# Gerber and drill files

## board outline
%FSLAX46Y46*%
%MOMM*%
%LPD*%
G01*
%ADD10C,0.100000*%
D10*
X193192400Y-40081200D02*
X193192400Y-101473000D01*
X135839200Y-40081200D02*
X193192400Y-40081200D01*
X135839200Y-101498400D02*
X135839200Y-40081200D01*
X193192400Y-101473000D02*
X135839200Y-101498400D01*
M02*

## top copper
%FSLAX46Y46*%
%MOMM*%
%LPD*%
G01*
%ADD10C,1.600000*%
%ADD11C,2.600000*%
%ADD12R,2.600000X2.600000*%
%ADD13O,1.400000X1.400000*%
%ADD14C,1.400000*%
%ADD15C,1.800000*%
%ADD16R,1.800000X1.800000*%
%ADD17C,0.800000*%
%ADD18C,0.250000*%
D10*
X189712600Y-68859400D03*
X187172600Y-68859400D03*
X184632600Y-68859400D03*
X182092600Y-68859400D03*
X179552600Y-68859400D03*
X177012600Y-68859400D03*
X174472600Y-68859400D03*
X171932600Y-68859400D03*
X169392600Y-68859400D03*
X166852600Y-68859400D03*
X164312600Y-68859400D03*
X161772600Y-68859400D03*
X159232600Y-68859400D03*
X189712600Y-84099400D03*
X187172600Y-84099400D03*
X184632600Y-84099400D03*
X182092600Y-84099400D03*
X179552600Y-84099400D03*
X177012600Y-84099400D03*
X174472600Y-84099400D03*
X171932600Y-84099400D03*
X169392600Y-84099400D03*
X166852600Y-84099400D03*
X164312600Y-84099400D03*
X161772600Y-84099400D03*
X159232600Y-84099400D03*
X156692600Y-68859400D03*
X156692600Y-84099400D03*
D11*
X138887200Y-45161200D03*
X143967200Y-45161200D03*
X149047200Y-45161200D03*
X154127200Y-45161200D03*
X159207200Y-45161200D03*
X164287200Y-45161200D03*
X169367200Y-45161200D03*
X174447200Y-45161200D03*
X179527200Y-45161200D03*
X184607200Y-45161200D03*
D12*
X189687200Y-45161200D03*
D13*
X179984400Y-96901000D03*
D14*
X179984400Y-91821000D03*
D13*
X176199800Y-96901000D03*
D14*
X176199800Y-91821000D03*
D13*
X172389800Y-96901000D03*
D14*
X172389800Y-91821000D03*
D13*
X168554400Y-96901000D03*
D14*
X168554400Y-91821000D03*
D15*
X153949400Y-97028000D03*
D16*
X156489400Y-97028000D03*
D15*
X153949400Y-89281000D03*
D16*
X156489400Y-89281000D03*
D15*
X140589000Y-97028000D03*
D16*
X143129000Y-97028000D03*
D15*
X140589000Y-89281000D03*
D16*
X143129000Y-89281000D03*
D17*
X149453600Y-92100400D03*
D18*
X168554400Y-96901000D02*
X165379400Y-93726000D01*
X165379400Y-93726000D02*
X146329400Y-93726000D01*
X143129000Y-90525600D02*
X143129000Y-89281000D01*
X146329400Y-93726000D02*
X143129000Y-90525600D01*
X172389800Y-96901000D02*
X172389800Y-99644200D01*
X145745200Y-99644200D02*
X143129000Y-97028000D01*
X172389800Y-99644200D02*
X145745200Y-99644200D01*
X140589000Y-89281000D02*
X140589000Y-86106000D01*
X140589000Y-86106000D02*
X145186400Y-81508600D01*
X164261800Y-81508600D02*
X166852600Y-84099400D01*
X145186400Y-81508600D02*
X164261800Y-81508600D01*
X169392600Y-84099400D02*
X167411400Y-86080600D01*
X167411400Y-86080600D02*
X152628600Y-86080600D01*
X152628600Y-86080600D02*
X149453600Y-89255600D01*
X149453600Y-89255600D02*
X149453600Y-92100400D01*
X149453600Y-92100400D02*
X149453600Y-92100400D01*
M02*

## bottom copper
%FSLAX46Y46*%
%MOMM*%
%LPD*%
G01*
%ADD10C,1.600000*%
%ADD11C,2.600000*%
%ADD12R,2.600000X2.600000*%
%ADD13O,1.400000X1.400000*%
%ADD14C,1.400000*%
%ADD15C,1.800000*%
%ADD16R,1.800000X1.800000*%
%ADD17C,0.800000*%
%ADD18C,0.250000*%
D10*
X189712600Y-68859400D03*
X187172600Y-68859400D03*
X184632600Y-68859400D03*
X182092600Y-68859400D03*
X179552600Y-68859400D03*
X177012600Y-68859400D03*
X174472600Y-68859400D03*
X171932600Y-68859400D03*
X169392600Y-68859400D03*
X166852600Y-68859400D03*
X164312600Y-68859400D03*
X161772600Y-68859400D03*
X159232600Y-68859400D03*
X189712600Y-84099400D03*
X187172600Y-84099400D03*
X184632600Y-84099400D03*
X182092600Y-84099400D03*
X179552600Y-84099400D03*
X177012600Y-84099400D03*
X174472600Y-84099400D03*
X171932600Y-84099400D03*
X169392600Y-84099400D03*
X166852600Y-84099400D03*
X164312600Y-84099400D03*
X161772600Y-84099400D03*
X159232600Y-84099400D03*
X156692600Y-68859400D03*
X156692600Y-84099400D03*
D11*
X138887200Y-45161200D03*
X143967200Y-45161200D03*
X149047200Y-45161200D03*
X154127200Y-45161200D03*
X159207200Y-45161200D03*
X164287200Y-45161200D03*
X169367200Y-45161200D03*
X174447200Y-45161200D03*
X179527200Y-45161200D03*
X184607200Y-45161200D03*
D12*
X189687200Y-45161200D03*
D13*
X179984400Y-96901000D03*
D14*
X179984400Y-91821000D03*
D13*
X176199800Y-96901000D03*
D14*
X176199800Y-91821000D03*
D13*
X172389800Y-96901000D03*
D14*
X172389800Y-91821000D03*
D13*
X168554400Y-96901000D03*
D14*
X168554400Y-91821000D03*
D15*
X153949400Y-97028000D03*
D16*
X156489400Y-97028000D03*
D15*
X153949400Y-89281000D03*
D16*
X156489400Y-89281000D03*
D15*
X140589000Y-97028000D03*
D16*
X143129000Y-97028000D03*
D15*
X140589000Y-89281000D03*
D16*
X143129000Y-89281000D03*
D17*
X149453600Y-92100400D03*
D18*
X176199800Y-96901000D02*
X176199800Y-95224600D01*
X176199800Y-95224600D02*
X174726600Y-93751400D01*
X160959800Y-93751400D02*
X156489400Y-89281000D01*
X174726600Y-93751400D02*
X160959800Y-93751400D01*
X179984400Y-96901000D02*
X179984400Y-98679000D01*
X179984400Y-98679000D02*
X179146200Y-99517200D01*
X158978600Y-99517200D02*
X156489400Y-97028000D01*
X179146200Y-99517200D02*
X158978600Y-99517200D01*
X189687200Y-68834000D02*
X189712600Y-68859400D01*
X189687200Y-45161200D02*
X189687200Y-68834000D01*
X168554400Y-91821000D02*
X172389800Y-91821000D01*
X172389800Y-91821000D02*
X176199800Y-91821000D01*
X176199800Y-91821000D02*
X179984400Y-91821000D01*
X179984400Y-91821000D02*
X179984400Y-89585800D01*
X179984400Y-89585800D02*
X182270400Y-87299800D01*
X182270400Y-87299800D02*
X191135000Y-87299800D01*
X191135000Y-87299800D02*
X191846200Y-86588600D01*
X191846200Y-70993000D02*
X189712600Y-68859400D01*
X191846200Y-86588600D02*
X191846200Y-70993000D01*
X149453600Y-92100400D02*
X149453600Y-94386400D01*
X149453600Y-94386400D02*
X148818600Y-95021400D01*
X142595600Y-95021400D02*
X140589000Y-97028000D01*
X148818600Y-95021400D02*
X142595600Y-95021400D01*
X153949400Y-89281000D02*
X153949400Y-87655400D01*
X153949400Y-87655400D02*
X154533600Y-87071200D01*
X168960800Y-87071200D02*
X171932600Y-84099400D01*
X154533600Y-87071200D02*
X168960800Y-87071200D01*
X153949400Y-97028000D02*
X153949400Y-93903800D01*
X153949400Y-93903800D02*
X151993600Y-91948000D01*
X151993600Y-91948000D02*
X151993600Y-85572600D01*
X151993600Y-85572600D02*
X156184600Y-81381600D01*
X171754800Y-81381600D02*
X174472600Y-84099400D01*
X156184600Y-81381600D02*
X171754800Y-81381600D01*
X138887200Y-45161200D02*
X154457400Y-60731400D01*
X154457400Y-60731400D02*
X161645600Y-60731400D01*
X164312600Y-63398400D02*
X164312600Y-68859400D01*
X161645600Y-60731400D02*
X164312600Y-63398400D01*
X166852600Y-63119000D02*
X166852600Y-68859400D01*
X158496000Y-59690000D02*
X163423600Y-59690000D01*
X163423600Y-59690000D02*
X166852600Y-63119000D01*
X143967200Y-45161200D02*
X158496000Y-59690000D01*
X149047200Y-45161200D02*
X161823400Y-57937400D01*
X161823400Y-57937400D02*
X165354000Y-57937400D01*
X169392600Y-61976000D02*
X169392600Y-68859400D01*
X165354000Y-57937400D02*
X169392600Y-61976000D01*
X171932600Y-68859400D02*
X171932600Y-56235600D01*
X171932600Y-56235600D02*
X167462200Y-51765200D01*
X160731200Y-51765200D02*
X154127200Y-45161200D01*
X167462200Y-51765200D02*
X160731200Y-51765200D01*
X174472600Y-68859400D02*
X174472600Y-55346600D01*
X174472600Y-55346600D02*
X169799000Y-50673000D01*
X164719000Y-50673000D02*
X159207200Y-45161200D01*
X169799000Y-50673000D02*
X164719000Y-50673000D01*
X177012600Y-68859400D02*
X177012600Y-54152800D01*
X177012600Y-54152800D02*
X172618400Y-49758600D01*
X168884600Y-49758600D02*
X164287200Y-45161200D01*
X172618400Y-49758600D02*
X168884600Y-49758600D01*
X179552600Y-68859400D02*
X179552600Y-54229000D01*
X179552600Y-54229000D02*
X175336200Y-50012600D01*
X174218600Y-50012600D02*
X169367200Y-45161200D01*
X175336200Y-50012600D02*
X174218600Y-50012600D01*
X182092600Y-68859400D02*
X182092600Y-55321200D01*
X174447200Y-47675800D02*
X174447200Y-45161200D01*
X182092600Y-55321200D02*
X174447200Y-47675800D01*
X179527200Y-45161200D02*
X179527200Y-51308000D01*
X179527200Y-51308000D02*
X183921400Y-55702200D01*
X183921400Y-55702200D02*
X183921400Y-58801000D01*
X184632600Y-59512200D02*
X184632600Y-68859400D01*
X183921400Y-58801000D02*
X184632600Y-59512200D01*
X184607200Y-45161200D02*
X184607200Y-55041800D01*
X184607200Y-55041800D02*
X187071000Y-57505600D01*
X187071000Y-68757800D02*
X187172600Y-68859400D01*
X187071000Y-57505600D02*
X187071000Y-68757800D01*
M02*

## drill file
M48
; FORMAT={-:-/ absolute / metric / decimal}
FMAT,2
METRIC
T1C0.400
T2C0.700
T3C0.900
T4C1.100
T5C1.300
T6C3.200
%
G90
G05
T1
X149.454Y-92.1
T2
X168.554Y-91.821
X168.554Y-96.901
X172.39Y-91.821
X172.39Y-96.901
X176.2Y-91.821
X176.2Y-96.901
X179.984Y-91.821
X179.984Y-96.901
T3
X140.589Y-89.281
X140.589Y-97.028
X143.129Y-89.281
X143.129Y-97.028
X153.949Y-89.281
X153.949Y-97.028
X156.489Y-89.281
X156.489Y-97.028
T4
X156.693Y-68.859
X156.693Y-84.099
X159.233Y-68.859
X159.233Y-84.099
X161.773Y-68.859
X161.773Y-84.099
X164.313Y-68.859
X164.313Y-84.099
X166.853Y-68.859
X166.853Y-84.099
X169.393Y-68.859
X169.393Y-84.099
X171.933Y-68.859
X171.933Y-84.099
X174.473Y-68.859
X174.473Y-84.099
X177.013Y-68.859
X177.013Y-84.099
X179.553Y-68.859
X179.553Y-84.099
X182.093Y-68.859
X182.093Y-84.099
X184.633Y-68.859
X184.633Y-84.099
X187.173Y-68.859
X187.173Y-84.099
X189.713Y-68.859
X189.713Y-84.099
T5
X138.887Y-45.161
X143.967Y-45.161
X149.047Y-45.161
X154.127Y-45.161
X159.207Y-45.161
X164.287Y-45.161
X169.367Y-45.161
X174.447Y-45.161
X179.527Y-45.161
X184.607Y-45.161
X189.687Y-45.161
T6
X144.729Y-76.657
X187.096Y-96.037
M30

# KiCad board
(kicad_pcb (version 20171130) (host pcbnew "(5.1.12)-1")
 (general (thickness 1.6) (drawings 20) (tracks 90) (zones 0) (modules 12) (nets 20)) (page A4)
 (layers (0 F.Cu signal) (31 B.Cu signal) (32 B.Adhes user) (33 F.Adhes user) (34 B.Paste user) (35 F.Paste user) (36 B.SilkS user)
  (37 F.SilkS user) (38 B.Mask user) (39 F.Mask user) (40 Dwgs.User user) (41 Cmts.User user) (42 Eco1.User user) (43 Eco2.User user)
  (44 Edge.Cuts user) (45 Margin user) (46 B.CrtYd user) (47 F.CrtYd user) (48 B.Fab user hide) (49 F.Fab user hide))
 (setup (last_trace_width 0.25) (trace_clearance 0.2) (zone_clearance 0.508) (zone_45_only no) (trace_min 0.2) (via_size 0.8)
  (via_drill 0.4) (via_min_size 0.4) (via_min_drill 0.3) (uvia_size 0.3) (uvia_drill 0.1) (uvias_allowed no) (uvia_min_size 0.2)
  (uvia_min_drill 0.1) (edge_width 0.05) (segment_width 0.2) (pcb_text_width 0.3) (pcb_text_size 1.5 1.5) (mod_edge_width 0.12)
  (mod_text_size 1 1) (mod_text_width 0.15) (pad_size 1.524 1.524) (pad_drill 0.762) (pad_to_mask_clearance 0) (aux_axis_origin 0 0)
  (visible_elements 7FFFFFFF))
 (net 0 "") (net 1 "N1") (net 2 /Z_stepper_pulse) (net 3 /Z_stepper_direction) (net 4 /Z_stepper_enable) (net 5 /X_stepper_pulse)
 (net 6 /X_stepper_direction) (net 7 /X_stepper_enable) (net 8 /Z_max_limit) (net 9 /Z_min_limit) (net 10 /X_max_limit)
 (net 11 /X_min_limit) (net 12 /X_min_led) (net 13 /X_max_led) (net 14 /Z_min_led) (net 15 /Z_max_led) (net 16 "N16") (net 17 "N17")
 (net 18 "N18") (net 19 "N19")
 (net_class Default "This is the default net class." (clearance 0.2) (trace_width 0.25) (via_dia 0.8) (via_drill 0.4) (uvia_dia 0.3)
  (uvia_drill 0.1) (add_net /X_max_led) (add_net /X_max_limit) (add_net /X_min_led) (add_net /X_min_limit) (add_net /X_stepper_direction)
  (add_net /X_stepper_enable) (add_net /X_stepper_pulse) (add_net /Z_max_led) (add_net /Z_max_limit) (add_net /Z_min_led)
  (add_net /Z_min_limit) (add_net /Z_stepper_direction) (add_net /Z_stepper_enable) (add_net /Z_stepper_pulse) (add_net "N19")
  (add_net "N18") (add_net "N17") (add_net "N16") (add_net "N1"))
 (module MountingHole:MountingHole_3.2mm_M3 (layer F.Cu) (at 144.7292 76.6572)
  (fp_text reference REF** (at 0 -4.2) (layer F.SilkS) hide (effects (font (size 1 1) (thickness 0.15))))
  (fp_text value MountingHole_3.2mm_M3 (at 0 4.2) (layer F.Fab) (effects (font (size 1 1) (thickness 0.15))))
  (pad 1 np_thru_hole circle (at 0 0) (size 3.2 3.2) (drill 3.2) (layers *.Cu *.Mask)))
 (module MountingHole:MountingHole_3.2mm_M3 (layer F.Cu) (at 187.0964 96.0374)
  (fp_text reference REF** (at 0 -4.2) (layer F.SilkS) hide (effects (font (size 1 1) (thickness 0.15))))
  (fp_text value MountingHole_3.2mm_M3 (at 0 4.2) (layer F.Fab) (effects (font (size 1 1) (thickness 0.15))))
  (pad 1 np_thru_hole circle (at 0 0) (size 3.2 3.2) (drill 3.2) (layers *.Cu *.Mask)))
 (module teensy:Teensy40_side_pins (layer F.Cu) (at 173.2026 76.4794 180)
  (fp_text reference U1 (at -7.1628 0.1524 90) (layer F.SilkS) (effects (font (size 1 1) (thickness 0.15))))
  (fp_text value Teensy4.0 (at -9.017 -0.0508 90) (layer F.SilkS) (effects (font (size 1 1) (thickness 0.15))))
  (pad 1 thru_hole circle (at -16.51 7.62 180) (size 1.6 1.6) (drill 1.1) (layers *.Cu *.Mask) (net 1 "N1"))
  (pad 2 thru_hole circle (at -13.97 7.62 180) (size 1.6 1.6) (drill 1.1) (layers *.Cu *.Mask) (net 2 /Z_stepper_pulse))
  (pad 3 thru_hole circle (at -11.43 7.62 180) (size 1.6 1.6) (drill 1.1) (layers *.Cu *.Mask) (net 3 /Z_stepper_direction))
  (pad 4 thru_hole circle (at -8.89 7.62 180) (size 1.6 1.6) (drill 1.1) (layers *.Cu *.Mask) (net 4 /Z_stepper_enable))
  (pad 5 thru_hole circle (at -6.35 7.62 180) (size 1.6 1.6) (drill 1.1) (layers *.Cu *.Mask) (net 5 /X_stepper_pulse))
  (pad 6 thru_hole circle (at -3.81 7.62 180) (size 1.6 1.6) (drill 1.1) (layers *.Cu *.Mask) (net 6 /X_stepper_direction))
  (pad 7 thru_hole circle (at -1.27 7.62 180) (size 1.6 1.6) (drill 1.1) (layers *.Cu *.Mask) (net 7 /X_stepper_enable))
  (pad 8 thru_hole circle (at 1.27 7.62 180) (size 1.6 1.6) (drill 1.1) (layers *.Cu *.Mask) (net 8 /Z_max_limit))
  (pad 9 thru_hole circle (at 3.81 7.62 180) (size 1.6 1.6) (drill 1.1) (layers *.Cu *.Mask) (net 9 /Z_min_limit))
  (pad 10 thru_hole circle (at 6.35 7.62 180) (size 1.6 1.6) (drill 1.1) (layers *.Cu *.Mask) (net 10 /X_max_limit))
  (pad 11 thru_hole circle (at 8.89 7.62 180) (size 1.6 1.6) (drill 1.1) (layers *.Cu *.Mask) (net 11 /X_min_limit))
  (pad 12 thru_hole circle (at 11.43 7.62 180) (size 1.6 1.6) (drill 1.1) (layers *.Cu *.Mask))
  (pad 13 thru_hole circle (at 13.97 7.62 180) (size 1.6 1.6) (drill 1.1) (layers *.Cu *.Mask))
  (pad 33 thru_hole circle (at -16.51 -7.62 180) (size 1.6 1.6) (drill 1.1) (layers *.Cu *.Mask))
  (pad 32 thru_hole circle (at -13.97 -7.62 180) (size 1.6 1.6) (drill 1.1) (layers *.Cu *.Mask))
  (pad 31 thru_hole circle (at -11.43 -7.62 180) (size 1.6 1.6) (drill 1.1) (layers *.Cu *.Mask))
  (pad 30 thru_hole circle (at -8.89 -7.62 180) (size 1.6 1.6) (drill 1.1) (layers *.Cu *.Mask))
  (pad 29 thru_hole circle (at -6.35 -7.62 180) (size 1.6 1.6) (drill 1.1) (layers *.Cu *.Mask))
  (pad 28 thru_hole circle (at -3.81 -7.62 180) (size 1.6 1.6) (drill 1.1) (layers *.Cu *.Mask))
  (pad 27 thru_hole circle (at -1.27 -7.62 180) (size 1.6 1.6) (drill 1.1) (layers *.Cu *.Mask) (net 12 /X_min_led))
  (pad 26 thru_hole circle (at 1.27 -7.62 180) (size 1.6 1.6) (drill 1.1) (layers *.Cu *.Mask) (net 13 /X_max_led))
  (pad 25 thru_hole circle (at 3.81 -7.62 180) (size 1.6 1.6) (drill 1.1) (layers *.Cu *.Mask) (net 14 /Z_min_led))
  (pad 24 thru_hole circle (at 6.35 -7.62 180) (size 1.6 1.6) (drill 1.1) (layers *.Cu *.Mask) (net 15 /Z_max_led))
  (pad 23 thru_hole circle (at 8.89 -7.62 180) (size 1.6 1.6) (drill 1.1) (layers *.Cu *.Mask))
  (pad 22 thru_hole circle (at 11.43 -7.62 180) (size 1.6 1.6) (drill 1.1) (layers *.Cu *.Mask))
  (pad 21 thru_hole circle (at 13.97 -7.62 180) (size 1.6 1.6) (drill 1.1) (layers *.Cu *.Mask))
  (pad 14 thru_hole circle (at 16.51 7.62 180) (size 1.6 1.6) (drill 1.1) (layers *.Cu *.Mask))
  (pad 20 thru_hole circle (at 16.51 -7.62 180) (size 1.6 1.6) (drill 1.1) (layers *.Cu *.Mask)))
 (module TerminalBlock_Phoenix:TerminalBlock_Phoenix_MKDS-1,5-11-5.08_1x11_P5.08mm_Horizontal (layer F.Cu) (at 189.6872 45.1612 180)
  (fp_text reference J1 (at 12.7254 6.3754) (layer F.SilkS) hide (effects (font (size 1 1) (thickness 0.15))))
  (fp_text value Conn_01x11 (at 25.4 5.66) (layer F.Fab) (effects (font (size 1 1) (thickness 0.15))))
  (pad 11 thru_hole circle (at 50.8 0 180) (size 2.6 2.6) (drill 1.3) (layers *.Cu *.Mask) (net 11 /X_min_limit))
  (pad 10 thru_hole circle (at 45.72 0 180) (size 2.6 2.6) (drill 1.3) (layers *.Cu *.Mask) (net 10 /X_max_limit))
  (pad 9 thru_hole circle (at 40.64 0 180) (size 2.6 2.6) (drill 1.3) (layers *.Cu *.Mask) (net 9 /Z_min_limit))
  (pad 8 thru_hole circle (at 35.56 0 180) (size 2.6 2.6) (drill 1.3) (layers *.Cu *.Mask) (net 8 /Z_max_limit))
  (pad 7 thru_hole circle (at 30.48 0 180) (size 2.6 2.6) (drill 1.3) (layers *.Cu *.Mask) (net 7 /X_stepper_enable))
  (pad 6 thru_hole circle (at 25.4 0 180) (size 2.6 2.6) (drill 1.3) (layers *.Cu *.Mask) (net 6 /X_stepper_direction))
  (pad 5 thru_hole circle (at 20.32 0 180) (size 2.6 2.6) (drill 1.3) (layers *.Cu *.Mask) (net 5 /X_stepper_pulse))
  (pad 4 thru_hole circle (at 15.24 0 180) (size 2.6 2.6) (drill 1.3) (layers *.Cu *.Mask) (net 4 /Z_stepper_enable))
  (pad 3 thru_hole circle (at 10.16 0 180) (size 2.6 2.6) (drill 1.3) (layers *.Cu *.Mask) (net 3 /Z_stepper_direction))
  (pad 2 thru_hole circle (at 5.08 0 180) (size 2.6 2.6) (drill 1.3) (layers *.Cu *.Mask) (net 2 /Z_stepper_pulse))
  (pad 1 thru_hole rect (at 0 0 180) (size 2.6 2.6) (drill 1.3) (layers *.Cu *.Mask) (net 1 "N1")))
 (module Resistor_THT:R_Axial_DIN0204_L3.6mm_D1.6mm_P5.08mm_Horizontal (layer F.Cu) (at 179.9844 91.821 270)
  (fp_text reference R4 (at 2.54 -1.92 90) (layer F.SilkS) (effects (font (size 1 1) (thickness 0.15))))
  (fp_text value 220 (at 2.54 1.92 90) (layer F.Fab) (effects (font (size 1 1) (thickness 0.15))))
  (pad 2 thru_hole oval (at 5.08 0 270) (size 1.4 1.4) (drill 0.7) (layers *.Cu *.Mask) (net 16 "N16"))
  (pad 1 thru_hole circle (at 0 0 270) (size 1.4 1.4) (drill 0.7) (layers *.Cu *.Mask) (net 1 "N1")))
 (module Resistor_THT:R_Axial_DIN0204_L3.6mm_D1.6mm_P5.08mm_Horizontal (layer F.Cu) (at 176.1998 91.821 270)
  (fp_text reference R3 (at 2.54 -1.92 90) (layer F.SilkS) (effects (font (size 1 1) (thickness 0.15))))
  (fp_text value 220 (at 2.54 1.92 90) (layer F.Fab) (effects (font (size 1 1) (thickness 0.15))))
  (pad 2 thru_hole oval (at 5.08 0 270) (size 1.4 1.4) (drill 0.7) (layers *.Cu *.Mask) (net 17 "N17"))
  (pad 1 thru_hole circle (at 0 0 270) (size 1.4 1.4) (drill 0.7) (layers *.Cu *.Mask) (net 1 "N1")))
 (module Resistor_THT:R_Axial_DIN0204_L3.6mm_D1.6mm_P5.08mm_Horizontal (layer F.Cu) (at 172.3898 91.821 270)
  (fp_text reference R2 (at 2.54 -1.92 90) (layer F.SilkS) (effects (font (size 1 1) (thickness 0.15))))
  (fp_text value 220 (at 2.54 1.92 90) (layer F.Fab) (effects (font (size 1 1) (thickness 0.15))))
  (pad 2 thru_hole oval (at 5.08 0 270) (size 1.4 1.4) (drill 0.7) (layers *.Cu *.Mask) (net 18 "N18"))
  (pad 1 thru_hole circle (at 0 0 270) (size 1.4 1.4) (drill 0.7) (layers *.Cu *.Mask) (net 1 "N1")))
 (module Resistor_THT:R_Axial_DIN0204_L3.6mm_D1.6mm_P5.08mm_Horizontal (layer F.Cu) (at 168.5544 91.821 270)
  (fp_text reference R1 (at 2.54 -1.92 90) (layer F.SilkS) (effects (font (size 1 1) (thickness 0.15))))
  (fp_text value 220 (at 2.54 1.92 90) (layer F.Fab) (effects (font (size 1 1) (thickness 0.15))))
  (pad 2 thru_hole oval (at 5.08 0 270) (size 1.4 1.4) (drill 0.7) (layers *.Cu *.Mask) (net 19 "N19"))
  (pad 1 thru_hole circle (at 0 0 270) (size 1.4 1.4) (drill 0.7) (layers *.Cu *.Mask) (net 1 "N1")))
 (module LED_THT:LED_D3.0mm (layer F.Cu) (at 156.4894 97.028 180)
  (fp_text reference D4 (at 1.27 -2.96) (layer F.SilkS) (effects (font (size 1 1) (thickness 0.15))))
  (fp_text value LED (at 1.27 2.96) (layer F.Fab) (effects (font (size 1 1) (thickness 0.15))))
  (pad 2 thru_hole circle (at 2.54 0 180) (size 1.8 1.8) (drill 0.9) (layers *.Cu *.Mask) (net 12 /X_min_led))
  (pad 1 thru_hole rect (at 0 0 180) (size 1.8 1.8) (drill 0.9) (layers *.Cu *.Mask) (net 16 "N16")))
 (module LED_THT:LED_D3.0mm (layer F.Cu) (at 156.4894 89.281 180)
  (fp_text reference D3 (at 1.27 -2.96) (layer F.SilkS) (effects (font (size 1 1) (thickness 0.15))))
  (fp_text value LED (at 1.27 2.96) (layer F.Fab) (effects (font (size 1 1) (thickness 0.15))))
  (pad 2 thru_hole circle (at 2.54 0 180) (size 1.8 1.8) (drill 0.9) (layers *.Cu *.Mask) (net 13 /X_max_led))
  (pad 1 thru_hole rect (at 0 0 180) (size 1.8 1.8) (drill 0.9) (layers *.Cu *.Mask) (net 17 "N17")))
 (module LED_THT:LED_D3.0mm (layer F.Cu) (at 143.129 97.028 180)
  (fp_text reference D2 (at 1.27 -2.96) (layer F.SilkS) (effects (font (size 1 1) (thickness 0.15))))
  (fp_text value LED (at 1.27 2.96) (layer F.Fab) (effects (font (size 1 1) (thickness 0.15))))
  (pad 2 thru_hole circle (at 2.54 0 180) (size 1.8 1.8) (drill 0.9) (layers *.Cu *.Mask) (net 14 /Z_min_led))
  (pad 1 thru_hole rect (at 0 0 180) (size 1.8 1.8) (drill 0.9) (layers *.Cu *.Mask) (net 18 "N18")))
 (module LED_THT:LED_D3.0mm (layer F.Cu) (at 143.129 89.281 180)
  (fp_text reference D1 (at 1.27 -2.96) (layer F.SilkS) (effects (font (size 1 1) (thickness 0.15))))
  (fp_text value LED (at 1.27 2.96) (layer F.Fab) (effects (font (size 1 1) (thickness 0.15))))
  (pad 2 thru_hole circle (at 2.54 0 180) (size 1.8 1.8) (drill 0.9) (layers *.Cu *.Mask) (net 15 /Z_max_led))
  (pad 1 thru_hole rect (at 0 0 180) (size 1.8 1.8) (drill 0.9) (layers *.Cu *.Mask) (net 19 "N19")))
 (gr_line (start 193.1924 40.0812) (end 193.1924 101.473) (layer Edge.Cuts) (width 0.1))
 (gr_line (start 135.8392 40.0812) (end 193.1924 40.0812) (layer Edge.Cuts) (width 0.1))
 (gr_line (start 135.8392 101.4984) (end 135.8392 40.0812) (layer Edge.Cuts) (width 0.1))
 (gr_line (start 193.1924 101.473) (end 135.8392 101.4984) (layer Edge.Cuts) (width 0.1))
 (segment (start 168.5544 96.901) (end 165.3794 93.726) (width 0.25) (layer F.Cu) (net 19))
 (segment (start 165.3794 93.726) (end 146.3294 93.726) (width 0.25) (layer F.Cu) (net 19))
 (segment (start 143.129 90.5256) (end 143.129 89.281) (width 0.25) (layer F.Cu) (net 19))
 (segment (start 146.3294 93.726) (end 143.129 90.5256) (width 0.25) (layer F.Cu) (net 19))
 (segment (start 172.3898 96.901) (end 172.3898 99.6442) (width 0.25) (layer F.Cu) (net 18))
 (segment (start 145.7452 99.6442) (end 143.129 97.028) (width 0.25) (layer F.Cu) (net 18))
 (segment (start 172.3898 99.6442) (end 145.7452 99.6442) (width 0.25) (layer F.Cu) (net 18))
 (segment (start 176.1998 96.901) (end 176.1998 95.2246) (width 0.25) (layer B.Cu) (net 17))
 (segment (start 176.1998 95.2246) (end 174.7266 93.7514) (width 0.25) (layer B.Cu) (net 17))
 (segment (start 160.9598 93.7514) (end 156.4894 89.281) (width 0.25) (layer B.Cu) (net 17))
 (segment (start 174.7266 93.7514) (end 160.9598 93.7514) (width 0.25) (layer B.Cu) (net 17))
 (segment (start 179.9844 96.901) (end 179.9844 98.679) (width 0.25) (layer B.Cu) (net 16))
 (segment (start 179.9844 98.679) (end 179.1462 99.5172) (width 0.25) (layer B.Cu) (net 16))
 (segment (start 158.9786 99.5172) (end 156.4894 97.028) (width 0.25) (layer B.Cu) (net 16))
 (segment (start 179.1462 99.5172) (end 158.9786 99.5172) (width 0.25) (layer B.Cu) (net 16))
 (segment (start 189.6872 68.834) (end 189.7126 68.8594) (width 0.25) (layer B.Cu) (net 1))
 (segment (start 189.6872 45.1612) (end 189.6872 68.834) (width 0.25) (layer B.Cu) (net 1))
 (segment (start 168.5544 91.821) (end 172.3898 91.821) (width 0.25) (layer B.Cu) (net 1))
 (segment (start 172.3898 91.821) (end 176.1998 91.821) (width 0.25) (layer B.Cu) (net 1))
 (segment (start 176.1998 91.821) (end 179.9844 91.821) (width 0.25) (layer B.Cu) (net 1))
 (segment (start 179.9844 91.821) (end 179.9844 89.5858) (width 0.25) (layer B.Cu) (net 1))
 (segment (start 179.9844 89.5858) (end 182.2704 87.2998) (width 0.25) (layer B.Cu) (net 1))
 (segment (start 182.2704 87.2998) (end 191.135 87.2998) (width 0.25) (layer B.Cu) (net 1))
 (segment (start 191.135 87.2998) (end 191.8462 86.5886) (width 0.25) (layer B.Cu) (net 1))
 (segment (start 191.8462 70.993) (end 189.7126 68.8594) (width 0.25) (layer B.Cu) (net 1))
 (segment (start 191.8462 86.5886) (end 191.8462 70.993) (width 0.25) (layer B.Cu) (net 1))
 (segment (start 140.589 89.281) (end 140.589 86.106) (width 0.25) (layer F.Cu) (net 15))
 (segment (start 140.589 86.106) (end 145.1864 81.5086) (width 0.25) (layer F.Cu) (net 15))
 (segment (start 164.2618 81.5086) (end 166.8526 84.0994) (width 0.25) (layer F.Cu) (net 15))
 (segment (start 145.1864 81.5086) (end 164.2618 81.5086) (width 0.25) (layer F.Cu) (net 15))
 (segment (start 169.3926 84.0994) (end 167.4114 86.0806) (width 0.25) (layer F.Cu) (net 14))
 (segment (start 167.4114 86.0806) (end 152.6286 86.0806) (width 0.25) (layer F.Cu) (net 14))
 (segment (start 152.6286 86.0806) (end 149.4536 89.2556) (width 0.25) (layer F.Cu) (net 14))
 (segment (start 149.4536 89.2556) (end 149.4536 92.1004) (width 0.25) (layer F.Cu) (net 14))
 (segment (start 149.4536 92.1004) (end 149.4536 92.1004) (width 0.25) (layer F.Cu) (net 14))
 (via (at 149.4536 92.1004) (size 0.8) (drill 0.4) (layers F.Cu B.Cu) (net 14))
 (segment (start 149.4536 92.1004) (end 149.4536 94.3864) (width 0.25) (layer B.Cu) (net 14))
 (segment (start 149.4536 94.3864) (end 148.8186 95.0214) (width 0.25) (layer B.Cu) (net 14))
 (segment (start 142.5956 95.0214) (end 140.589 97.028) (width 0.25) (layer B.Cu) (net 14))
 (segment (start 148.8186 95.0214) (end 142.5956 95.0214) (width 0.25) (layer B.Cu) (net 14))
 (segment (start 153.9494 89.281) (end 153.9494 87.6554) (width 0.25) (layer B.Cu) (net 13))
 (segment (start 153.9494 87.6554) (end 154.5336 87.0712) (width 0.25) (layer B.Cu) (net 13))
 (segment (start 168.9608 87.0712) (end 171.9326 84.0994) (width 0.25) (layer B.Cu) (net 13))
 (segment (start 154.5336 87.0712) (end 168.9608 87.0712) (width 0.25) (layer B.Cu) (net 13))
 (segment (start 153.9494 97.028) (end 153.9494 93.9038) (width 0.25) (layer B.Cu) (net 12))
 (segment (start 153.9494 93.9038) (end 151.9936 91.948) (width 0.25) (layer B.Cu) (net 12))
 (segment (start 151.9936 91.948) (end 151.9936 85.5726) (width 0.25) (layer B.Cu) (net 12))
 (segment (start 151.9936 85.5726) (end 156.1846 81.3816) (width 0.25) (layer B.Cu) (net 12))
 (segment (start 171.7548 81.3816) (end 174.4726 84.0994) (width 0.25) (layer B.Cu) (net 12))
 (segment (start 156.1846 81.3816) (end 171.7548 81.3816) (width 0.25) (layer B.Cu) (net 12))
 (segment (start 138.8872 45.1612) (end 154.4574 60.7314) (width 0.25) (layer B.Cu) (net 11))
 (segment (start 154.4574 60.7314) (end 161.6456 60.7314) (width 0.25) (layer B.Cu) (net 11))
 (segment (start 164.3126 63.3984) (end 164.3126 68.8594) (width 0.25) (layer B.Cu) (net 11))
 (segment (start 161.6456 60.7314) (end 164.3126 63.3984) (width 0.25) (layer B.Cu) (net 11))
 (segment (start 166.8526 63.119) (end 166.8526 68.8594) (width 0.25) (layer B.Cu) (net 10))
 (segment (start 158.496 59.69) (end 163.4236 59.69) (width 0.25) (layer B.Cu) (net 10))
 (segment (start 163.4236 59.69) (end 166.8526 63.119) (width 0.25) (layer B.Cu) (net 10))
 (segment (start 143.9672 45.1612) (end 158.496 59.69) (width 0.25) (layer B.Cu) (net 10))
 (segment (start 149.0472 45.1612) (end 161.8234 57.9374) (width 0.25) (layer B.Cu) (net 9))
 (segment (start 161.8234 57.9374) (end 165.354 57.9374) (width 0.25) (layer B.Cu) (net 9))
 (segment (start 169.3926 61.976) (end 169.3926 68.8594) (width 0.25) (layer B.Cu) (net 9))
 (segment (start 165.354 57.9374) (end 169.3926 61.976) (width 0.25) (layer B.Cu) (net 9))
 (segment (start 171.9326 68.8594) (end 171.9326 56.2356) (width 0.25) (layer B.Cu) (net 8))
 (segment (start 171.9326 56.2356) (end 167.4622 51.7652) (width 0.25) (layer B.Cu) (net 8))
 (segment (start 160.7312 51.7652) (end 154.1272 45.1612) (width 0.25) (layer B.Cu) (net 8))
 (segment (start 167.4622 51.7652) (end 160.7312 51.7652) (width 0.25) (layer B.Cu) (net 8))
 (segment (start 174.4726 68.8594) (end 174.4726 55.3466) (width 0.25) (layer B.Cu) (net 7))
 (segment (start 174.4726 55.3466) (end 169.799 50.673) (width 0.25) (layer B.Cu) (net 7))
 (segment (start 164.719 50.673) (end 159.2072 45.1612) (width 0.25) (layer B.Cu) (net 7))
 (segment (start 169.799 50.673) (end 164.719 50.673) (width 0.25) (layer B.Cu) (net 7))
 (segment (start 177.0126 68.8594) (end 177.0126 54.1528) (width 0.25) (layer B.Cu) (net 6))
 (segment (start 177.0126 54.1528) (end 172.6184 49.7586) (width 0.25) (layer B.Cu) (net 6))
 (segment (start 168.8846 49.7586) (end 164.2872 45.1612) (width 0.25) (layer B.Cu) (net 6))
 (segment (start 172.6184 49.7586) (end 168.8846 49.7586) (width 0.25) (layer B.Cu) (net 6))
 (segment (start 179.5526 68.8594) (end 179.5526 54.229) (width 0.25) (layer B.Cu) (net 5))
 (segment (start 179.5526 54.229) (end 175.3362 50.0126) (width 0.25) (layer B.Cu) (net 5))
 (segment (start 174.2186 50.0126) (end 169.3672 45.1612) (width 0.25) (layer B.Cu) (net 5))
 (segment (start 175.3362 50.0126) (end 174.2186 50.0126) (width 0.25) (layer B.Cu) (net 5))
 (segment (start 182.0926 68.8594) (end 182.0926 55.3212) (width 0.25) (layer B.Cu) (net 4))
 (segment (start 174.4472 47.6758) (end 174.4472 45.1612) (width 0.25) (layer B.Cu) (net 4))
 (segment (start 182.0926 55.3212) (end 174.4472 47.6758) (width 0.25) (layer B.Cu) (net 4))
 (segment (start 179.5272 45.1612) (end 179.5272 51.308) (width 0.25) (layer B.Cu) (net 3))
 (segment (start 179.5272 51.308) (end 183.9214 55.7022) (width 0.25) (layer B.Cu) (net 3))
 (segment (start 183.9214 55.7022) (end 183.9214 58.801) (width 0.25) (layer B.Cu) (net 3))
 (segment (start 184.6326 59.5122) (end 184.6326 68.8594) (width 0.25) (layer B.Cu) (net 3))
 (segment (start 183.9214 58.801) (end 184.6326 59.5122) (width 0.25) (layer B.Cu) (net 3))
 (segment (start 184.6072 45.1612) (end 184.6072 55.0418) (width 0.25) (layer B.Cu) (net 2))
 (segment (start 184.6072 55.0418) (end 187.071 57.5056) (width 0.25) (layer B.Cu) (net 2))
 (segment (start 187.071 68.7578) (end 187.1726 68.8594) (width 0.25) (layer B.Cu) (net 2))
 (segment (start 187.071 57.5056) (end 187.071 68.7578) (width 0.25) (layer B.Cu) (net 2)))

